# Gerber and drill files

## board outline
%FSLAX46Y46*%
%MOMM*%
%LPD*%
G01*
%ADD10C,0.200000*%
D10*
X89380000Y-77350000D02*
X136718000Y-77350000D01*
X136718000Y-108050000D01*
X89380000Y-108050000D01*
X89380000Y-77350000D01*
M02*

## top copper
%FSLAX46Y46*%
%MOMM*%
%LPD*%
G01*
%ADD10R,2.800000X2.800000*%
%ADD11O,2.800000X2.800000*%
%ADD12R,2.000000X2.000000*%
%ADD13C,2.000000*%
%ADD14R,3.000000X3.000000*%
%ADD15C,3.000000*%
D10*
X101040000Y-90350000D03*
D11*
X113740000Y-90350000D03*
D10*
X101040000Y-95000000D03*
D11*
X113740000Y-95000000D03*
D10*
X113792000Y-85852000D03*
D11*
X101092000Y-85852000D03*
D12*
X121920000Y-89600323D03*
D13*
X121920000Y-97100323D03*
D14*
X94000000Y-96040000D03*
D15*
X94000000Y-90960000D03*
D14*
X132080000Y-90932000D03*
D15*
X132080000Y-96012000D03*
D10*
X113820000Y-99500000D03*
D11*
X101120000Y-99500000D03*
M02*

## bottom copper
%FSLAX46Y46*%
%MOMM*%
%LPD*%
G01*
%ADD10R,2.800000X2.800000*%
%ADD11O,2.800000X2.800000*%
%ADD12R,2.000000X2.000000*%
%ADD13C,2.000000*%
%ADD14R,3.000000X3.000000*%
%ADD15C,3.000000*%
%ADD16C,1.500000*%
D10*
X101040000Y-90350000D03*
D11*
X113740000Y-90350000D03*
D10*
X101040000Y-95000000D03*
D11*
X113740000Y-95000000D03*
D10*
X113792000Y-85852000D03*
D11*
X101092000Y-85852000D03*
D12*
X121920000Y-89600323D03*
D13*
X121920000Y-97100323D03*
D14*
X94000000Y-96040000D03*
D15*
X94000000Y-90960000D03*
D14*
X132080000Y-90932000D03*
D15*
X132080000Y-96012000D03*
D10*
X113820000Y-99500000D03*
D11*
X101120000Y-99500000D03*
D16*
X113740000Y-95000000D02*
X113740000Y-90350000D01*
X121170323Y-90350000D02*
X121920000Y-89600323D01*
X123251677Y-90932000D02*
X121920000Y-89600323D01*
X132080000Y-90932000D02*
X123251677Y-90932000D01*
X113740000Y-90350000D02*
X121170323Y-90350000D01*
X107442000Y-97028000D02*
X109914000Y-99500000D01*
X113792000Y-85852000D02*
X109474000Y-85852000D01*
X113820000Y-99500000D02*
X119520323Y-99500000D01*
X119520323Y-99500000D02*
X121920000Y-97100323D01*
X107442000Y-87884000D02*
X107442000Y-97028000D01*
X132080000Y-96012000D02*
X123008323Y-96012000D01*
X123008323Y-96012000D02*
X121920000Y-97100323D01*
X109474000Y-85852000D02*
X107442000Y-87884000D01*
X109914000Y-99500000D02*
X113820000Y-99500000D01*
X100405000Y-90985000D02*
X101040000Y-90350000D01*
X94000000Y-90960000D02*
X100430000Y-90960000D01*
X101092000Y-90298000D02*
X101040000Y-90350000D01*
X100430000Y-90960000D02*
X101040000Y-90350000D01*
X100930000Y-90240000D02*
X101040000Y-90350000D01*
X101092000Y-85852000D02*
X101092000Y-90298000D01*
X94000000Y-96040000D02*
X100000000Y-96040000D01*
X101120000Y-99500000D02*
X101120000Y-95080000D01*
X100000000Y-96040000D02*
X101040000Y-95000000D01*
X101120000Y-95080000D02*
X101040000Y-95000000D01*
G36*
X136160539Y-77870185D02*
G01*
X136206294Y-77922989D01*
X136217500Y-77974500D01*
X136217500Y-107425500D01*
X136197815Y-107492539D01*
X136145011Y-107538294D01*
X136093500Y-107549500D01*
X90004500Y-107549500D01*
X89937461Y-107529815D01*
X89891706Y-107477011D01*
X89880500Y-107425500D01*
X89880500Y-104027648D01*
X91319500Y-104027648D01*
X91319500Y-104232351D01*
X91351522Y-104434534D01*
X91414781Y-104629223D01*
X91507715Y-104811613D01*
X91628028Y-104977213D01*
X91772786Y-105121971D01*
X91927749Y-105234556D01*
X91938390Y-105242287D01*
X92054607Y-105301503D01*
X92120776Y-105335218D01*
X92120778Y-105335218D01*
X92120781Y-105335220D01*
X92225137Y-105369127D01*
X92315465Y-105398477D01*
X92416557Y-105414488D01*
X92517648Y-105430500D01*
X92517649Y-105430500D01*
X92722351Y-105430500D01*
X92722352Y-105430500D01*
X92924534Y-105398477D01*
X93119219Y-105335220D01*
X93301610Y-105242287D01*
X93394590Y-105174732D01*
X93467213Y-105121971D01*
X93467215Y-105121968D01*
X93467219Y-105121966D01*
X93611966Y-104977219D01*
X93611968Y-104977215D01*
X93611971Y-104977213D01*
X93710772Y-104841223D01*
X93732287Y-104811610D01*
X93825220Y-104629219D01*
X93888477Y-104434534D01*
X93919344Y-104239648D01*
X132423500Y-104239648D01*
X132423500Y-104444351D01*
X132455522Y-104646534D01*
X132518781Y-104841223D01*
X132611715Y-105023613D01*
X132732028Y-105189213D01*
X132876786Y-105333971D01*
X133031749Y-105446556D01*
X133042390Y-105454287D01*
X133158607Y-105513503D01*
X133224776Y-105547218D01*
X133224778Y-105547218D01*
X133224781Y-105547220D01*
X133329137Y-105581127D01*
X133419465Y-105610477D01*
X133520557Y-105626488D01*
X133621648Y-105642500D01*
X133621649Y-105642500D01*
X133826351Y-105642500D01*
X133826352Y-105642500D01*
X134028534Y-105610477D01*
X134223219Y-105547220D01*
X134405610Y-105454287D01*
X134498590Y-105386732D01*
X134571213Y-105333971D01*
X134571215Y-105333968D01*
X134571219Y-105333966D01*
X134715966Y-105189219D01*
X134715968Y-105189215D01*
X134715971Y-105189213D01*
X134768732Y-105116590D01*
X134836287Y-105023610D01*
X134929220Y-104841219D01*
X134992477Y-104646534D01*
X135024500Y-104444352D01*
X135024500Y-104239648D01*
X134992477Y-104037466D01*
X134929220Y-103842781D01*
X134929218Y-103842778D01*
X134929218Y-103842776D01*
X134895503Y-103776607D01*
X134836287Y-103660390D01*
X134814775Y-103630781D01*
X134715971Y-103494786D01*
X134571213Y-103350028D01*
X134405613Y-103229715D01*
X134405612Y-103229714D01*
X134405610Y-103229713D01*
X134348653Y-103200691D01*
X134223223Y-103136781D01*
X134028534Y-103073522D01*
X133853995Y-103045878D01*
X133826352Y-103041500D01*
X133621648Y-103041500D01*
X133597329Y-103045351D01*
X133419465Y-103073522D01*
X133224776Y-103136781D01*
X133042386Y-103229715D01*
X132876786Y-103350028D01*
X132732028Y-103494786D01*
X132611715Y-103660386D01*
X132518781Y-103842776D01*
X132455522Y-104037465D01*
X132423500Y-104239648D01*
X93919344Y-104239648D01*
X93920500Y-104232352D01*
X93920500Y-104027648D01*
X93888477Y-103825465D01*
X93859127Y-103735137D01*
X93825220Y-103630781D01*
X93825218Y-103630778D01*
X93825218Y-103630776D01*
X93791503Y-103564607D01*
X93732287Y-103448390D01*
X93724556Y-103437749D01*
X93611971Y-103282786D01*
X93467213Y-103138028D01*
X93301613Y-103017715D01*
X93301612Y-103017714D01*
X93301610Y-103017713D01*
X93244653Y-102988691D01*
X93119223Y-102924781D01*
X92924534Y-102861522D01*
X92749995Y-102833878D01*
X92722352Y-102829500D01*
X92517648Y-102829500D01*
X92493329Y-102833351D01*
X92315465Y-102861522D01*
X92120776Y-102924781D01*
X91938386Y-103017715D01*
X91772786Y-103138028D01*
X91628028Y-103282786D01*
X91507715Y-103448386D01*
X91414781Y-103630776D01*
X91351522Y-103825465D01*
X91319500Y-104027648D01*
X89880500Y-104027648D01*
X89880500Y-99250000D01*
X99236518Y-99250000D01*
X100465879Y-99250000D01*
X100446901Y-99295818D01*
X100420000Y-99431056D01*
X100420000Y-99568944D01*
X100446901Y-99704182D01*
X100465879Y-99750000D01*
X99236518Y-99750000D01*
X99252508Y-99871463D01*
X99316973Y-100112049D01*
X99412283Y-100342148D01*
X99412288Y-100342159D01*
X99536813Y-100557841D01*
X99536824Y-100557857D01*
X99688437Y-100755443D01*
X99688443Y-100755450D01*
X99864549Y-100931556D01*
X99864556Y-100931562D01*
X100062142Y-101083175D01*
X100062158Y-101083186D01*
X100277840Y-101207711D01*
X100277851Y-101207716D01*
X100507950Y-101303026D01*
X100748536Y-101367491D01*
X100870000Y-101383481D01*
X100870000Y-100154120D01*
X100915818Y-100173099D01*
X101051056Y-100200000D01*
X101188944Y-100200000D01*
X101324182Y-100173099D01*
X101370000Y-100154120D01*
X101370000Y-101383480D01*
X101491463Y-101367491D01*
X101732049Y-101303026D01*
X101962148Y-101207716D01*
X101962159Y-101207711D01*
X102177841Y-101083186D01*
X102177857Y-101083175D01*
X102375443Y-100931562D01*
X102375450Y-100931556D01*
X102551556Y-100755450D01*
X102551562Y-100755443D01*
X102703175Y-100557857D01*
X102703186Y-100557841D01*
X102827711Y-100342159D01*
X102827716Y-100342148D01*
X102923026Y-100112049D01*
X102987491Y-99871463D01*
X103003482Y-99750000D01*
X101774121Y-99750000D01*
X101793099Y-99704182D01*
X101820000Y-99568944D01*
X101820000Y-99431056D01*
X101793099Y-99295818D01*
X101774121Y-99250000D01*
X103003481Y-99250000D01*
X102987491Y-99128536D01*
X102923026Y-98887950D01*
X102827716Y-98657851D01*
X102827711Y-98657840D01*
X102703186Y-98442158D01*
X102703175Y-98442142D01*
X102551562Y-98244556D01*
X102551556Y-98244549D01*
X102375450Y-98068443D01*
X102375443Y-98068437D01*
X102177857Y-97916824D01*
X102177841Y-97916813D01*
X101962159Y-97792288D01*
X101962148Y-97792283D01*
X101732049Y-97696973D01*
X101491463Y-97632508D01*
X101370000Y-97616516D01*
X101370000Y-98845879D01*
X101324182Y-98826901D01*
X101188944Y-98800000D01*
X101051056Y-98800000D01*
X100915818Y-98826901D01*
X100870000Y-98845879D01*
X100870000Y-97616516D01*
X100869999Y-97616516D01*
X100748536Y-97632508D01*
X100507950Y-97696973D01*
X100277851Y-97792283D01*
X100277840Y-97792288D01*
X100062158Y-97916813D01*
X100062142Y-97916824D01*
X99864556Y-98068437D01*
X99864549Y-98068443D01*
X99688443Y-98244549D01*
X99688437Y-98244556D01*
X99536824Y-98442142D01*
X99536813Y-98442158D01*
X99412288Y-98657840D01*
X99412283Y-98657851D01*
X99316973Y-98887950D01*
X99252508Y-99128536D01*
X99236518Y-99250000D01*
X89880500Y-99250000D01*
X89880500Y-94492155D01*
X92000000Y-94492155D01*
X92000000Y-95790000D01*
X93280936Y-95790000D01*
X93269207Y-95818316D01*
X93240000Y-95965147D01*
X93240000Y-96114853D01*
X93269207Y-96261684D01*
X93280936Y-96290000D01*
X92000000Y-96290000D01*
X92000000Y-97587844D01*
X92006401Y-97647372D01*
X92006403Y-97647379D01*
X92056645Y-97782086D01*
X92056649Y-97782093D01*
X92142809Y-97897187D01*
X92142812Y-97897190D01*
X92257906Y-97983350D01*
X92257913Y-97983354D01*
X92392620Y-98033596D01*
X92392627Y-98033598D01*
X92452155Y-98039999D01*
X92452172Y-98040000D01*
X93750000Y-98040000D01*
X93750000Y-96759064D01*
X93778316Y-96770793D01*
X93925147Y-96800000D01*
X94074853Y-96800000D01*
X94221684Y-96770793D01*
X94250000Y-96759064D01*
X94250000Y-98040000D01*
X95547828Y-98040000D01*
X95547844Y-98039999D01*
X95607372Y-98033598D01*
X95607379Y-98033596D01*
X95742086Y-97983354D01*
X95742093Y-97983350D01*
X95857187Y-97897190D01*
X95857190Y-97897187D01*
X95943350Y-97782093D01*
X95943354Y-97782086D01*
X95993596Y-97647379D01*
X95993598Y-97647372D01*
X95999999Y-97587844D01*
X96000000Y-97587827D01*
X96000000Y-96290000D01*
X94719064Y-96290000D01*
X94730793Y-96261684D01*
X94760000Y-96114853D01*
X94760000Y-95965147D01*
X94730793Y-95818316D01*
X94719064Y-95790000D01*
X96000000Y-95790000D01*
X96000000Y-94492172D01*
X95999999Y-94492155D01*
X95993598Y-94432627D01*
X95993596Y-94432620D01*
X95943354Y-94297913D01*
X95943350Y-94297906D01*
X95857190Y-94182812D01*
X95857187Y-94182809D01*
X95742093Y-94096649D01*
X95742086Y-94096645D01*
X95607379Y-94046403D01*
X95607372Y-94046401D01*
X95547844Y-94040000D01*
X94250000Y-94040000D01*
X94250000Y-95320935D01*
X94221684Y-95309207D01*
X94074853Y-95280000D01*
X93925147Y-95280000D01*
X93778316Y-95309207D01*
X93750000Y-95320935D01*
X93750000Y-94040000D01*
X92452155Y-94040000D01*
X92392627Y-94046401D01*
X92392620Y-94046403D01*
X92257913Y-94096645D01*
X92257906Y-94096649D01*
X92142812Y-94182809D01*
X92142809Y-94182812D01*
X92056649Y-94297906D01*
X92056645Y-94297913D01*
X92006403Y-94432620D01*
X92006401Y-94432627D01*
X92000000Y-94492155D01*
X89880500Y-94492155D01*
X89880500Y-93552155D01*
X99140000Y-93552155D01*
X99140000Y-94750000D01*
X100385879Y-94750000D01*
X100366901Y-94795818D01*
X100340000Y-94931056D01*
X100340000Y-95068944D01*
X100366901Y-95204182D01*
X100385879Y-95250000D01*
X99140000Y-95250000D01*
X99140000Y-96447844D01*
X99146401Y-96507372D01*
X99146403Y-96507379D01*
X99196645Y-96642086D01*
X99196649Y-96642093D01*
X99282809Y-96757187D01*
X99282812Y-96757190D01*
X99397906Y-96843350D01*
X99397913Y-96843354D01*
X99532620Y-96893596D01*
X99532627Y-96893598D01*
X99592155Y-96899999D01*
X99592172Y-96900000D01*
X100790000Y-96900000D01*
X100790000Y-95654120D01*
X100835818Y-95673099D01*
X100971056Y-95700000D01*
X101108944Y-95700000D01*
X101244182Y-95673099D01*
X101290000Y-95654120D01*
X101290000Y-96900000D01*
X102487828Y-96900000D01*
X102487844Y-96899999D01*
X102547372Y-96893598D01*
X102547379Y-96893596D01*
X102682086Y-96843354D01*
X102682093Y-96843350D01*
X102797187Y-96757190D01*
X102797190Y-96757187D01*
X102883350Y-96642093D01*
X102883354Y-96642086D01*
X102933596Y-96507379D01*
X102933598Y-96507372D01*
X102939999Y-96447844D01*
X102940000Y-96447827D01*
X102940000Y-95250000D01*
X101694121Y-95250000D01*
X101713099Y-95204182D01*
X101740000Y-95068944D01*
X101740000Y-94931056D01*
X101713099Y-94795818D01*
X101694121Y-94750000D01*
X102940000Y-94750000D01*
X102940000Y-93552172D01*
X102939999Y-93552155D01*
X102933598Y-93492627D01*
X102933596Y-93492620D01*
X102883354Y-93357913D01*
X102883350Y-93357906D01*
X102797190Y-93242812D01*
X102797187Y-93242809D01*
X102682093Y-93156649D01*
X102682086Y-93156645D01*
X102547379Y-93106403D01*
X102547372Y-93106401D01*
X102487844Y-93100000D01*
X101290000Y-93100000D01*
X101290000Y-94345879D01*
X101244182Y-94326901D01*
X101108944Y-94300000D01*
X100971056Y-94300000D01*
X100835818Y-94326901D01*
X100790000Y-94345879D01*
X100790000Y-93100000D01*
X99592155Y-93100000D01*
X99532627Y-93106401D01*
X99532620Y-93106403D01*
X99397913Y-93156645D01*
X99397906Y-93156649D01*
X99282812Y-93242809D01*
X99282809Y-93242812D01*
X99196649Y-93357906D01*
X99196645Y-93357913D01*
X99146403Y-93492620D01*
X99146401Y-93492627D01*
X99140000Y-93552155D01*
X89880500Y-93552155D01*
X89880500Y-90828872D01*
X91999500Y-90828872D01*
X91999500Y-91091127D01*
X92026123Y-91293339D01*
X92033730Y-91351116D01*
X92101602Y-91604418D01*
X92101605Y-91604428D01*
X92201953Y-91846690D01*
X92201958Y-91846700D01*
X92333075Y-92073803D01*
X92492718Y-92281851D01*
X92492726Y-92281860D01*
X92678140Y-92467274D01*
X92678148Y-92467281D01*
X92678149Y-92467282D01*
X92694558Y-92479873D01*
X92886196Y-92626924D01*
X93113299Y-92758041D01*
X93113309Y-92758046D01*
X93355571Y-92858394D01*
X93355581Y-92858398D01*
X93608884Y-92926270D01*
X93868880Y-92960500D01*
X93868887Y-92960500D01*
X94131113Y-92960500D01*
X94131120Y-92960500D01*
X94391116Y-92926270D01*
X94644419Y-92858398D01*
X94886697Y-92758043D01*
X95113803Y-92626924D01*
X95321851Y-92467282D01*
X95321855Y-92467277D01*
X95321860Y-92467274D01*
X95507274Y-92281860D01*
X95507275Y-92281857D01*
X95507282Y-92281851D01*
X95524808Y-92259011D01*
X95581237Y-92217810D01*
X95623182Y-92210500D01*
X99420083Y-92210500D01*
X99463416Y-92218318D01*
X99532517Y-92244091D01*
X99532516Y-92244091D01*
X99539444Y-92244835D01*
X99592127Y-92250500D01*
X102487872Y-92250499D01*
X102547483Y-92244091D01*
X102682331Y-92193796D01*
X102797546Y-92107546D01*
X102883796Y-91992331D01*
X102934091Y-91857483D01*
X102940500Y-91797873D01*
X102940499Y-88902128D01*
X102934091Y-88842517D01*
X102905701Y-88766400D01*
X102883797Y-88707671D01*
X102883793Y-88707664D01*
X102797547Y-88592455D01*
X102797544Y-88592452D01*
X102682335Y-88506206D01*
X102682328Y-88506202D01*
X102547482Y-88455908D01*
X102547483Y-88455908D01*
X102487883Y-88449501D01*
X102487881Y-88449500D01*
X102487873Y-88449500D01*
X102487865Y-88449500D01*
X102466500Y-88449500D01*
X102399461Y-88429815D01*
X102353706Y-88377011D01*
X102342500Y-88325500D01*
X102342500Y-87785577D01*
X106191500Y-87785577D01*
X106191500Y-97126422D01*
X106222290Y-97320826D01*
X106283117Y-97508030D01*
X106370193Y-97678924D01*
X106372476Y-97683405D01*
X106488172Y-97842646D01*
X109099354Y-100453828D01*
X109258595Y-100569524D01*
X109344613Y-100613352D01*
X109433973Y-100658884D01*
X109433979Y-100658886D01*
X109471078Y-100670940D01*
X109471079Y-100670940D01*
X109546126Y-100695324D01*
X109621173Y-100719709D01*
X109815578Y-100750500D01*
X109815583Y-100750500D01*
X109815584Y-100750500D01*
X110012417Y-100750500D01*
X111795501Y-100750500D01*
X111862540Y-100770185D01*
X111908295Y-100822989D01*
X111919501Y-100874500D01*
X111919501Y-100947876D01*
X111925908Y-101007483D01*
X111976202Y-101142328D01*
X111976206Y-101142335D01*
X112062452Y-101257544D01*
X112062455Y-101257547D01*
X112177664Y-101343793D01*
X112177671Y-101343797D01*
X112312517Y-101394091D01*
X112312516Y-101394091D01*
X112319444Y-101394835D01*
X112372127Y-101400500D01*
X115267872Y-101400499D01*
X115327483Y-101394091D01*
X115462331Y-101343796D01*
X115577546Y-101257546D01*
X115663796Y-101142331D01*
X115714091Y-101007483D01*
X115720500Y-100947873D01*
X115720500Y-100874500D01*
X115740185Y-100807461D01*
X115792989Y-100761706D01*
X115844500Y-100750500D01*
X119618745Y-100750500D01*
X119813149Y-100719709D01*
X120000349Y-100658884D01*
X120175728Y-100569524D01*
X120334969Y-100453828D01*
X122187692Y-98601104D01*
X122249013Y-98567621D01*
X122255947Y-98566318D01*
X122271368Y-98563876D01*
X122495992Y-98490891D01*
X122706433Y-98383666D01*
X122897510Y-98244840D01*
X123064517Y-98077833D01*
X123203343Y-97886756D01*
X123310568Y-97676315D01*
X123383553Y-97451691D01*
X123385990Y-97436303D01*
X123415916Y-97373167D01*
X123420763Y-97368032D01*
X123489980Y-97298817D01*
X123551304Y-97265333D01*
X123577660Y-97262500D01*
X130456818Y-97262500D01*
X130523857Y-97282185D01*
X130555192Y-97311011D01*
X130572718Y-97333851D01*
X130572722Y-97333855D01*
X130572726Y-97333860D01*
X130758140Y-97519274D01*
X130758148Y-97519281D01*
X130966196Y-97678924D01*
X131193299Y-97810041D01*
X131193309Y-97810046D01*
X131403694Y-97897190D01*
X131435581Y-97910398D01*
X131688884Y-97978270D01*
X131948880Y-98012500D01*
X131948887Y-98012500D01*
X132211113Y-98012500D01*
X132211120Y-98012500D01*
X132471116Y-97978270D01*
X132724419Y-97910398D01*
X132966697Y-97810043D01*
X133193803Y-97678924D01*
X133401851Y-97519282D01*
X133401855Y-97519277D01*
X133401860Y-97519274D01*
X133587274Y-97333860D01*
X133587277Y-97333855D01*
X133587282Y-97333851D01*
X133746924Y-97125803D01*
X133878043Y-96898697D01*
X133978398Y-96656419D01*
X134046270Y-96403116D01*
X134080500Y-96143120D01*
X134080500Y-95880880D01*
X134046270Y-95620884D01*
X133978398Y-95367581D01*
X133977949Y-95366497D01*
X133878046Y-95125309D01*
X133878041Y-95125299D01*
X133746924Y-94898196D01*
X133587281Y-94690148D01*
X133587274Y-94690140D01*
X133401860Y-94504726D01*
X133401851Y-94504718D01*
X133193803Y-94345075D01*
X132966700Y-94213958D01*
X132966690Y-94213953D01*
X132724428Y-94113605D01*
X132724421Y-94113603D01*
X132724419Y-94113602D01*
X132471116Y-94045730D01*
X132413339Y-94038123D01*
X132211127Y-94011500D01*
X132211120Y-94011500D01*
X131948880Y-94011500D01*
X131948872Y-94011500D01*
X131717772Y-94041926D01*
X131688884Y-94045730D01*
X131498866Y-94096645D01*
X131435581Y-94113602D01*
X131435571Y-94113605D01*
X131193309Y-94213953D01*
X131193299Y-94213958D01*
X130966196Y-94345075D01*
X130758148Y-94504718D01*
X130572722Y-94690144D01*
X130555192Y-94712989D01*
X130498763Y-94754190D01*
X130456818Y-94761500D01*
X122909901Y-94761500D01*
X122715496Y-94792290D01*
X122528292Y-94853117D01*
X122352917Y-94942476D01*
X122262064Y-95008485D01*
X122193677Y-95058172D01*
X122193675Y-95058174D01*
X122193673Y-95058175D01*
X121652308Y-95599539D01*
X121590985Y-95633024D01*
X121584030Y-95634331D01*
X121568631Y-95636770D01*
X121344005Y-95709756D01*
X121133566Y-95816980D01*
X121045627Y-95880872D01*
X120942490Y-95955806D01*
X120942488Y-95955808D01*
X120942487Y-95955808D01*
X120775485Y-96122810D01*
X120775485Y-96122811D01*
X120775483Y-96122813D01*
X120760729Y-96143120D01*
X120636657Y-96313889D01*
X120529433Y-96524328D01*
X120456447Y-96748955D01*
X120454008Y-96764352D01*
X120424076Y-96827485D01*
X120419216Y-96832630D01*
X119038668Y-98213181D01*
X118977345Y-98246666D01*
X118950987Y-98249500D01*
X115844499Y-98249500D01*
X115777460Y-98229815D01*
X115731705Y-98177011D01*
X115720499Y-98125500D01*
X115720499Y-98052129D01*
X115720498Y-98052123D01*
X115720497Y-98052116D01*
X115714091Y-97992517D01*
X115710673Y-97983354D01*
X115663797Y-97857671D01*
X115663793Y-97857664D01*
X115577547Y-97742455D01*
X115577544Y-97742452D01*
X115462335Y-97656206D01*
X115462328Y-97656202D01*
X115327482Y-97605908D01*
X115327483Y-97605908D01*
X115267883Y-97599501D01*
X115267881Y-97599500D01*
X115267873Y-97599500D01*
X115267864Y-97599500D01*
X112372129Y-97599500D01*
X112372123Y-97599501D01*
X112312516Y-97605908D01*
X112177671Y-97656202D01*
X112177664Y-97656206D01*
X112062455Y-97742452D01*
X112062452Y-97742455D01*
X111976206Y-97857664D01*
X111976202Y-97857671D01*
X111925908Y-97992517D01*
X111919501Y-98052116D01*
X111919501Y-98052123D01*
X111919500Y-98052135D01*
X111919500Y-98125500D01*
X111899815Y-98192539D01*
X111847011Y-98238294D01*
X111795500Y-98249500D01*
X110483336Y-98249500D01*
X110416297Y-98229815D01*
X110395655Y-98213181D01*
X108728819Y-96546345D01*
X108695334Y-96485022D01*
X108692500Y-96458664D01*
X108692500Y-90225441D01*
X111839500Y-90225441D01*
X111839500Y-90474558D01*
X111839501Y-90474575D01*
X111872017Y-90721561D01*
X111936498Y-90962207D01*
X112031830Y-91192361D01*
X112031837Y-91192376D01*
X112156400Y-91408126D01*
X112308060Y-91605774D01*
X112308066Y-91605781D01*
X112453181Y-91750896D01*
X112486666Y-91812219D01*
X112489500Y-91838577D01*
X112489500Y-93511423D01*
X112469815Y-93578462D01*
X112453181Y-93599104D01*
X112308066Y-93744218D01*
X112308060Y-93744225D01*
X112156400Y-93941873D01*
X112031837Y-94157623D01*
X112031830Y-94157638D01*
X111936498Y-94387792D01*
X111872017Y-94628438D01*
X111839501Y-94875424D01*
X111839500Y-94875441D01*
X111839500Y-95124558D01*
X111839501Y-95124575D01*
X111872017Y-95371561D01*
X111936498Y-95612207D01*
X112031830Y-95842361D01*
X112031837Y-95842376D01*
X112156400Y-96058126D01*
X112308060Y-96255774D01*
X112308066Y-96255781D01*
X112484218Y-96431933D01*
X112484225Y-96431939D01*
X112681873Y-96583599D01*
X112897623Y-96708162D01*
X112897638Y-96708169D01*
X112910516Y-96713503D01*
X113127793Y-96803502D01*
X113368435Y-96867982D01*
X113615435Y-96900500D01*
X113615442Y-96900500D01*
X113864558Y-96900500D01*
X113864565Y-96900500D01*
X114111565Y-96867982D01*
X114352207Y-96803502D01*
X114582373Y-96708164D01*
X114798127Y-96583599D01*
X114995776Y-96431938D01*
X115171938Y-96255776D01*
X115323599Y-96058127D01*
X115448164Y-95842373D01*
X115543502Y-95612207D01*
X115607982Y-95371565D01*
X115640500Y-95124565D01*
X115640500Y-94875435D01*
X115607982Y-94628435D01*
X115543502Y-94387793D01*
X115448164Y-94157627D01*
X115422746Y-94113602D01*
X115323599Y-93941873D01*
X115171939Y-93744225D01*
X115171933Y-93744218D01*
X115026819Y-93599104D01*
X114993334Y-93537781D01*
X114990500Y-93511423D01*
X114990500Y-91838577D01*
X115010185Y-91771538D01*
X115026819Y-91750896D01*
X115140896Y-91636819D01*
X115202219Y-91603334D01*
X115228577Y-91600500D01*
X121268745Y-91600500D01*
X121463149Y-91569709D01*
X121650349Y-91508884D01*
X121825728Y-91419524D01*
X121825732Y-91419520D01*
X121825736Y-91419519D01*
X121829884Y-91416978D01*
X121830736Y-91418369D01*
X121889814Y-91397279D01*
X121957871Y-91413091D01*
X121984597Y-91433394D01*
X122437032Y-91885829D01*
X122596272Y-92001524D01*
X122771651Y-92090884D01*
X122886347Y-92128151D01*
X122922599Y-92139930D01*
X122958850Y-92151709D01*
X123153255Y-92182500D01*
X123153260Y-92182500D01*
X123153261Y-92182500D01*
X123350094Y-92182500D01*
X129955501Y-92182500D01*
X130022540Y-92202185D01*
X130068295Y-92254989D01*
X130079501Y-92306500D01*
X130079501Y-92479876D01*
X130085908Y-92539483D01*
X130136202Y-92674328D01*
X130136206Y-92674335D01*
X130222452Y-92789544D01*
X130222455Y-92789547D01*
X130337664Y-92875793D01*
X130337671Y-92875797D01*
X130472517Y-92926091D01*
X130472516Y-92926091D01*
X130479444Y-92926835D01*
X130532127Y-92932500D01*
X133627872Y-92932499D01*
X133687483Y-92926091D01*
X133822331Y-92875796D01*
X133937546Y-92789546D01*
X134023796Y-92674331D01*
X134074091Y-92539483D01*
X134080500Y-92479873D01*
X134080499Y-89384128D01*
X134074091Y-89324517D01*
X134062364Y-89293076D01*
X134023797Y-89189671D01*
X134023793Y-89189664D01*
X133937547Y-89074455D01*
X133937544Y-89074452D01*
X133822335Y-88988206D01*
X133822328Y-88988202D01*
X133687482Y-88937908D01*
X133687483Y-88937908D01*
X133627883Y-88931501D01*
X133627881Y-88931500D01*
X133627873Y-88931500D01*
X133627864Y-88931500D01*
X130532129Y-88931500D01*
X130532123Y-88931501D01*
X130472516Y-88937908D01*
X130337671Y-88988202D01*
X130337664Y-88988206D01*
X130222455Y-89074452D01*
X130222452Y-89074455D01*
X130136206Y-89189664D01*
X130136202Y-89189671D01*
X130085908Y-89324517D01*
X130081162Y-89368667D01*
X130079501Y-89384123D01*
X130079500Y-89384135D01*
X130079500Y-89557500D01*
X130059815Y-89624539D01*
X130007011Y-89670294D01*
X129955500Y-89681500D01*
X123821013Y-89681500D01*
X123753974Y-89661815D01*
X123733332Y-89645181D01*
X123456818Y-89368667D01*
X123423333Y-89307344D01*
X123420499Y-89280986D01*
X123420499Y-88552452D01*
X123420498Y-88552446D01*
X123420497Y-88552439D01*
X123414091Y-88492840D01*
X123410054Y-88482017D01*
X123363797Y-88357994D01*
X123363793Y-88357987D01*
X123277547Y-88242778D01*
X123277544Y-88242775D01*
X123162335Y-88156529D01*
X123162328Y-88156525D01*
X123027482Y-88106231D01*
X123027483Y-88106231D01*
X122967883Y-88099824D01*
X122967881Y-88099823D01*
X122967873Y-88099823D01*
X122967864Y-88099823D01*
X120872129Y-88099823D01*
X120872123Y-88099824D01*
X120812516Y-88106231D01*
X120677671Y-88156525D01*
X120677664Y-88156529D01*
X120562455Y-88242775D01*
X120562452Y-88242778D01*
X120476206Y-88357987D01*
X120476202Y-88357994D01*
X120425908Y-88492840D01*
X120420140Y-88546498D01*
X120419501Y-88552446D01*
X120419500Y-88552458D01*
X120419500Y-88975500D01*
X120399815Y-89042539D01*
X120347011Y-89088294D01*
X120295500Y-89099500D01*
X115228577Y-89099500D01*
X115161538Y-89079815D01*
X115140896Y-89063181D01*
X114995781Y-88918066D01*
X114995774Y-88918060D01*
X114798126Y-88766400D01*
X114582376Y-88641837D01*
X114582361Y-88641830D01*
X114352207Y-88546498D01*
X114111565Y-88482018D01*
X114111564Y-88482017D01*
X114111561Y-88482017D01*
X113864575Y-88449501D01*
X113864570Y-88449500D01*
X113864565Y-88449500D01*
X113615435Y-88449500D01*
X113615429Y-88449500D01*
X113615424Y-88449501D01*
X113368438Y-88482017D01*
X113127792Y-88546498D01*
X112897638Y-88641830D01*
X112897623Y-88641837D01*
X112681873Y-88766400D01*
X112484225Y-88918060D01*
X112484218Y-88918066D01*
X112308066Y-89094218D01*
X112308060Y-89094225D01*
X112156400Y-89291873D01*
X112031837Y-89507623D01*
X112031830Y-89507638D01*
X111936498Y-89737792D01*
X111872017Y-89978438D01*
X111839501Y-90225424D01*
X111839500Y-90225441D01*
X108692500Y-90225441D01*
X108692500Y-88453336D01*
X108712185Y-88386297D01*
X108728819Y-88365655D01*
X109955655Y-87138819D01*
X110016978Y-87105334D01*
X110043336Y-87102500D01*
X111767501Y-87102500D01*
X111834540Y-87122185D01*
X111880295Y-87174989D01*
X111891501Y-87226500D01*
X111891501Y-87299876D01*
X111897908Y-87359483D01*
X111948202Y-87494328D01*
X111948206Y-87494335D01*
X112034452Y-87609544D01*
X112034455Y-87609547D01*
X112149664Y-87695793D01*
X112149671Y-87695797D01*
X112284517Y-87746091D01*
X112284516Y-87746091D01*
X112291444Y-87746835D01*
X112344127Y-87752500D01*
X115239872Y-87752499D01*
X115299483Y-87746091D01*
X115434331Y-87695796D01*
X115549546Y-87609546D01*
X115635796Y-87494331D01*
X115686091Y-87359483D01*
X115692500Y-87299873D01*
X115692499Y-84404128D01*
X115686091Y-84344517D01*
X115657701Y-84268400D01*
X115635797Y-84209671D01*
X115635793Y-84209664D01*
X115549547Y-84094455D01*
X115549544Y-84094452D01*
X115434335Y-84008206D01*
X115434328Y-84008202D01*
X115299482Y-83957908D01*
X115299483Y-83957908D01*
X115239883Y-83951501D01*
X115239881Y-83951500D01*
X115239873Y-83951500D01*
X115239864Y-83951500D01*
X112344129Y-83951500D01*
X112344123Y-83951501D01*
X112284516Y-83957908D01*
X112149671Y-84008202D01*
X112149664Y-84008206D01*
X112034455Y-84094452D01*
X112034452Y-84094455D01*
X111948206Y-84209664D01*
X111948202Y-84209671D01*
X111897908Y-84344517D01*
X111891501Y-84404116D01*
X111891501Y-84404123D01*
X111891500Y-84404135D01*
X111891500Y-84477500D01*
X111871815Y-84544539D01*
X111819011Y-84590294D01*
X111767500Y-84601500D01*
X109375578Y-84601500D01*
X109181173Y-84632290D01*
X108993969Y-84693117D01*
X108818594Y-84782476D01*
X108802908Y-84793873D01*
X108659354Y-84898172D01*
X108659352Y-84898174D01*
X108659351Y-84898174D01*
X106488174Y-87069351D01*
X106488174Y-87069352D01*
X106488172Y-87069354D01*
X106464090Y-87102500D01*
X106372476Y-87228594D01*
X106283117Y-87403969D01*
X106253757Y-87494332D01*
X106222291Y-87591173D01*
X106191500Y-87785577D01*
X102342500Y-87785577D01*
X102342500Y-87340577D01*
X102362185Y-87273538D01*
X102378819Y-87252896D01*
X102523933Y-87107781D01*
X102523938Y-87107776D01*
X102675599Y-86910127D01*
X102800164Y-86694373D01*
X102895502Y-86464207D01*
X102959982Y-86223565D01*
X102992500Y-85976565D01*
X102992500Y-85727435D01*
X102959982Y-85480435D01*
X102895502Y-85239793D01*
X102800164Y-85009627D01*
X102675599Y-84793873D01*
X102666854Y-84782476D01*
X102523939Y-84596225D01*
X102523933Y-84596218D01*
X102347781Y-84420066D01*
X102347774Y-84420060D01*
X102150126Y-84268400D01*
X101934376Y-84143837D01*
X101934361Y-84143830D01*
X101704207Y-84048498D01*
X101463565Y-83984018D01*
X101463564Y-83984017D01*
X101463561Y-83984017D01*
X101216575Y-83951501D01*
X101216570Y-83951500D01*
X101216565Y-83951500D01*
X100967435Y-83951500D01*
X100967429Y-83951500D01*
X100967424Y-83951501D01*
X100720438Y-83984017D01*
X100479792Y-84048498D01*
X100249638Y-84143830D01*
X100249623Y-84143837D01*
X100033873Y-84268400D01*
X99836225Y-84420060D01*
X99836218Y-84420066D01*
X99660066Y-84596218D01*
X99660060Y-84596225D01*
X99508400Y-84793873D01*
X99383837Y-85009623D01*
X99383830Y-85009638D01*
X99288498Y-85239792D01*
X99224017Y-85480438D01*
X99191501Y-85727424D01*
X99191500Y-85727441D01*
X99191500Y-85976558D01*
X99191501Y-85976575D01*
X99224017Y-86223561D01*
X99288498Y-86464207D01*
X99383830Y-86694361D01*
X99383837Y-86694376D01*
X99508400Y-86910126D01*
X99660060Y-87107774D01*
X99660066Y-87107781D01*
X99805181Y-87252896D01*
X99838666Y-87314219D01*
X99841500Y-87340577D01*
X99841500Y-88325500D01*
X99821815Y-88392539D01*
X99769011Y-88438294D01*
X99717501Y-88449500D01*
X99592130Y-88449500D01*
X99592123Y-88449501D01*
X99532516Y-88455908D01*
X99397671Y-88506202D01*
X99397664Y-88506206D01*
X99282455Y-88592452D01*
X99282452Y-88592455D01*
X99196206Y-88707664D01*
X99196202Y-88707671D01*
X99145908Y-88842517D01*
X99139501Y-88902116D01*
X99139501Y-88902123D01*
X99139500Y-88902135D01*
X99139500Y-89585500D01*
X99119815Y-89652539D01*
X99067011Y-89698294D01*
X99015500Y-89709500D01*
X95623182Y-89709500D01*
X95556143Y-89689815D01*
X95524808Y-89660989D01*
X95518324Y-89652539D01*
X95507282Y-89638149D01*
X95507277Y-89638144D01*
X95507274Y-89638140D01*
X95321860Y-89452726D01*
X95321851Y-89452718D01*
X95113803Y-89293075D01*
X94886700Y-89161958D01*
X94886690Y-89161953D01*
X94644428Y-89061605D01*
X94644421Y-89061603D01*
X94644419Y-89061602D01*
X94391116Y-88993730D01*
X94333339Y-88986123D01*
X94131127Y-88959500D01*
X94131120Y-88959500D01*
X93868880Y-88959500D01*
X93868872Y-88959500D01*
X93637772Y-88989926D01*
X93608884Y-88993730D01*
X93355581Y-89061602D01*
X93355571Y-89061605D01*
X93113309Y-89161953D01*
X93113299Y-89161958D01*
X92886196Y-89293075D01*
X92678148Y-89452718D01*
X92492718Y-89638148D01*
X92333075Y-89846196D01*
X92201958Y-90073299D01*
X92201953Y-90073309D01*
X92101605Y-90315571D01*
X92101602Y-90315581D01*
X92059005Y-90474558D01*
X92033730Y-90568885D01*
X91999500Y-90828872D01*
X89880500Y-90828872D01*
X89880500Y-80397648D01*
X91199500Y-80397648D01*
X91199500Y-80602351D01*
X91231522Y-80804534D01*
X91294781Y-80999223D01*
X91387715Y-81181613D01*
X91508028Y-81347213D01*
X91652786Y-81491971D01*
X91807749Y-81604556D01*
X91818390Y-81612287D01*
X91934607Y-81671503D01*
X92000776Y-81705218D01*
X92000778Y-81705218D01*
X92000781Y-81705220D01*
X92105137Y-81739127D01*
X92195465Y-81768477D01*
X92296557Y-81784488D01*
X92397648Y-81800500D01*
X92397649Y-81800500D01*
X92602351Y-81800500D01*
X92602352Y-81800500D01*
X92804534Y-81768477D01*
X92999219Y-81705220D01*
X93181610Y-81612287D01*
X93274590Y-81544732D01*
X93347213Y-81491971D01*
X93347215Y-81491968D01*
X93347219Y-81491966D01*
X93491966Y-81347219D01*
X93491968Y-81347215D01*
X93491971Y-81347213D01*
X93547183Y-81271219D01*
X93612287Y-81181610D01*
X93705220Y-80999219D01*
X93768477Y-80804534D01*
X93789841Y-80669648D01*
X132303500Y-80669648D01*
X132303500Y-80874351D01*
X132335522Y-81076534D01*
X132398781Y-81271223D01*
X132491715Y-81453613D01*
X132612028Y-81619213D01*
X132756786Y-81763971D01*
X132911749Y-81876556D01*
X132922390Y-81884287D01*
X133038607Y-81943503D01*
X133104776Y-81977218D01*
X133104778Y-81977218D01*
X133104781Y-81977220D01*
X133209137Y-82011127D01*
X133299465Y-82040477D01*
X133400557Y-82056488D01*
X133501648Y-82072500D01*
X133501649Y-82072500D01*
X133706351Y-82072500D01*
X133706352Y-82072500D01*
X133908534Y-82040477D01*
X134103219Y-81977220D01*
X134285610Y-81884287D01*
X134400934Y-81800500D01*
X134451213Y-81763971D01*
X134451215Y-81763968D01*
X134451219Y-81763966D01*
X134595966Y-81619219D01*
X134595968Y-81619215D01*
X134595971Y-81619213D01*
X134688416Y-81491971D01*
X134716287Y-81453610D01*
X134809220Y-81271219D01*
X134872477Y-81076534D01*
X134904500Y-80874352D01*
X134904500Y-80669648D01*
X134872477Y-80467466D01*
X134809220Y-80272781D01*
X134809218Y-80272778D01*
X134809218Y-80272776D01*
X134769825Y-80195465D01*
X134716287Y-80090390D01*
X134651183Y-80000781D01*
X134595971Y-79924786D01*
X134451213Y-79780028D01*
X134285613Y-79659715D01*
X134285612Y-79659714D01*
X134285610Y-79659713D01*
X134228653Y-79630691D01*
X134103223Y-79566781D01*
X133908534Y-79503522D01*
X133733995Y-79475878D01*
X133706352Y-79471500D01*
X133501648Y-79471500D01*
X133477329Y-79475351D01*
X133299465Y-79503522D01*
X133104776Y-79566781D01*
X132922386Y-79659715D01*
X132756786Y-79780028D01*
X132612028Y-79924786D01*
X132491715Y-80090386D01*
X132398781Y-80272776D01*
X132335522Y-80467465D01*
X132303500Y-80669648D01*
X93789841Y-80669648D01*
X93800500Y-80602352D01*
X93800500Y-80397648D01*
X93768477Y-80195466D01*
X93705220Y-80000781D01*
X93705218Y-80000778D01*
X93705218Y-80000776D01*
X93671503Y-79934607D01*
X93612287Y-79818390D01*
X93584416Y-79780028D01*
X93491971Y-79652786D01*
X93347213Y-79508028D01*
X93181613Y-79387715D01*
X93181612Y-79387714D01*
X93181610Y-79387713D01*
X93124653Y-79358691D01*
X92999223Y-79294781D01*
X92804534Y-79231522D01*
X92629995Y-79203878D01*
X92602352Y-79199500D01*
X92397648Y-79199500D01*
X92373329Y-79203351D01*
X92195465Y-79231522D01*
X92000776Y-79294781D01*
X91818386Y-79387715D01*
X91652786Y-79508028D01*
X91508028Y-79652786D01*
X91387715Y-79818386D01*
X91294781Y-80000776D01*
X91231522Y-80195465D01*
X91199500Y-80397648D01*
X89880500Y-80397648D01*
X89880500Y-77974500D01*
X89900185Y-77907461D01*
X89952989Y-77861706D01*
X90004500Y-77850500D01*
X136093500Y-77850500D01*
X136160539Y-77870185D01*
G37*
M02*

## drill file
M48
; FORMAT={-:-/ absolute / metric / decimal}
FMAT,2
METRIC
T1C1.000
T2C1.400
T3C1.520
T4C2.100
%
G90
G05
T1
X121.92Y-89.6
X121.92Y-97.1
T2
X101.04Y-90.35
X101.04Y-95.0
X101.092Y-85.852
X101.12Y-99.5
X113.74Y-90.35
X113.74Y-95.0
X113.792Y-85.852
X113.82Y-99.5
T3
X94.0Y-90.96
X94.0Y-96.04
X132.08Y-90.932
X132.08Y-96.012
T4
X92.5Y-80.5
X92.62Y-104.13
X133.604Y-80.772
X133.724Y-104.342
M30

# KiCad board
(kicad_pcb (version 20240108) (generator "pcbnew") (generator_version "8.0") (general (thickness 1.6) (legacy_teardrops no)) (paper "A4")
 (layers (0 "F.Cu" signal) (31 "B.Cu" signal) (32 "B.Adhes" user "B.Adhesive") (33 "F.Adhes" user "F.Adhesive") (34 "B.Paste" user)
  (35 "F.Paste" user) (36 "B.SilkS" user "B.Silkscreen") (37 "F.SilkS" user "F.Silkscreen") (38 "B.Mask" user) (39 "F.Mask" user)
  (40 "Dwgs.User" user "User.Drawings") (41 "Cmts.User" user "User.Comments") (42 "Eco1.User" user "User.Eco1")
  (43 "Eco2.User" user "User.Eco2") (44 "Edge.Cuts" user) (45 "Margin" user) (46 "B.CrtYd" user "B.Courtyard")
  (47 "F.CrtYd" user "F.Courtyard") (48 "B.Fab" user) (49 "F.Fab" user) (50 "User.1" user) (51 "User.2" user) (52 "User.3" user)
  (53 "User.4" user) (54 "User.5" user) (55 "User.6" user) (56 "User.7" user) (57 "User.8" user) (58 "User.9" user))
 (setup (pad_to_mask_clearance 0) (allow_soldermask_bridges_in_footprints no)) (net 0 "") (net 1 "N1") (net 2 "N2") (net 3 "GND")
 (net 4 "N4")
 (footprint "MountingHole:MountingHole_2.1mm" (layer "F.Cu") (at 133.604 80.772)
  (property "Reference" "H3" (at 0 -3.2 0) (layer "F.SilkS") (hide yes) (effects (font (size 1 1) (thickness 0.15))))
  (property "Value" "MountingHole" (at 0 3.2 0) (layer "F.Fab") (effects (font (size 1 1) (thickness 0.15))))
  (pad "" np_thru_hole circle (at 0 0) (size 2.1 2.1) (drill 2.1) (layers "*.Cu" "*.Mask")))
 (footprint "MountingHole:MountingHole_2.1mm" (layer "F.Cu") (at 92.5 80.5)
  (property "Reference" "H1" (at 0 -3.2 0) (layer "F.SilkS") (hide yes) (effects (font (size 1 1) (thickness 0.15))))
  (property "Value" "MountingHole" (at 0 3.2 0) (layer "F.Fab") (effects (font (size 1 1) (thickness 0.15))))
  (pad "" np_thru_hole circle (at 0 0) (size 2.1 2.1) (drill 2.1) (layers "*.Cu" "*.Mask")))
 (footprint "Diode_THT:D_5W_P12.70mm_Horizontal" (layer "F.Cu") (at 101.04 90.35)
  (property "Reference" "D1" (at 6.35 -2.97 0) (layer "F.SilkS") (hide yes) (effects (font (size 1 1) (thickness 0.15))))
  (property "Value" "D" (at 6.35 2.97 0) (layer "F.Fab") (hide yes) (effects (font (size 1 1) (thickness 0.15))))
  (pad "1" thru_hole rect (at 0 0) (size 2.8 2.8) (drill 1.4) (layers "*.Cu" "*.Mask") (remove_unused_layers no) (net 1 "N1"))
  (pad "2" thru_hole oval (at 12.7 0) (size 2.8 2.8) (drill 1.4) (layers "*.Cu" "*.Mask") (remove_unused_layers no) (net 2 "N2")))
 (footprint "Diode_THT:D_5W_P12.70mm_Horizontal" (layer "F.Cu") (at 101.04 95)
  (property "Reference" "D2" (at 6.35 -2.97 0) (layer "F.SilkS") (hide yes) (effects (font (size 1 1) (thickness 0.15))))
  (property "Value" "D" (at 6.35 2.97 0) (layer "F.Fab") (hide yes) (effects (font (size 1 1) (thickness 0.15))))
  (pad "1" thru_hole rect (at 0 0) (size 2.8 2.8) (drill 1.4) (layers "*.Cu" "*.Mask") (remove_unused_layers no) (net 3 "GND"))
  (pad "2" thru_hole oval (at 12.7 0) (size 2.8 2.8) (drill 1.4) (layers "*.Cu" "*.Mask") (remove_unused_layers no) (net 2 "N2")))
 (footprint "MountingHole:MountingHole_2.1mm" (layer "F.Cu") (at 92.62 104.13)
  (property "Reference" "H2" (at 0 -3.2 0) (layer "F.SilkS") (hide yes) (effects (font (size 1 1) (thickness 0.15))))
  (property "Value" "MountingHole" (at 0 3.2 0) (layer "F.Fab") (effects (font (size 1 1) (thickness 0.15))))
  (pad "" np_thru_hole circle (at 0 0) (size 2.1 2.1) (drill 2.1) (layers "*.Cu" "*.Mask")))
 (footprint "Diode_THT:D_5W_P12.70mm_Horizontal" (layer "F.Cu") (at 113.792 85.852 180)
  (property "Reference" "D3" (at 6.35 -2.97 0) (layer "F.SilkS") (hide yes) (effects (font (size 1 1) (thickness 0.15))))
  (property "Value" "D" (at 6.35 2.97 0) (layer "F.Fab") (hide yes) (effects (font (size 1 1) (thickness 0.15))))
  (pad "1" thru_hole rect (at 0 0 180) (size 2.8 2.8) (drill 1.4) (layers "*.Cu" "*.Mask") (remove_unused_layers no) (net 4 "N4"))
  (pad "2" thru_hole oval (at 12.7 0 180) (size 2.8 2.8) (drill 1.4) (layers "*.Cu" "*.Mask") (remove_unused_layers no) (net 1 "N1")))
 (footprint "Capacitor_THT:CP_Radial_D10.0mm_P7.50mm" (layer "F.Cu") (at 121.92 89.600323 -90)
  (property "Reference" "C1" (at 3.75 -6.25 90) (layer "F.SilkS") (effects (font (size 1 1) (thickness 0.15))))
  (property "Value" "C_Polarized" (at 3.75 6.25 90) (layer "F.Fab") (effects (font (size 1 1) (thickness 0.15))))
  (pad "1" thru_hole rect (at 0 0 270) (size 2 2) (drill 1) (layers "*.Cu" "*.Mask") (remove_unused_layers no) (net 2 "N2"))
  (pad "2" thru_hole circle (at 7.5 0 270) (size 2 2) (drill 1) (layers "*.Cu" "*.Mask") (remove_unused_layers no) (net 4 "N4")))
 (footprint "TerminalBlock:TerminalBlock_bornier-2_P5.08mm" (layer "F.Cu") (at 94 96.04 90)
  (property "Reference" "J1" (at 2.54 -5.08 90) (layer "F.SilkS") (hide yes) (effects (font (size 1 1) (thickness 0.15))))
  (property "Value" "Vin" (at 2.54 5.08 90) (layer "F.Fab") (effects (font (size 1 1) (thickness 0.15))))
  (pad "1" thru_hole rect (at 0 0 90) (size 3 3) (drill 1.52) (layers "*.Cu" "*.Mask") (remove_unused_layers no) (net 3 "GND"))
  (pad "2" thru_hole circle (at 5.08 0 90) (size 3 3) (drill 1.52) (layers "*.Cu" "*.Mask") (remove_unused_layers no) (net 1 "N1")))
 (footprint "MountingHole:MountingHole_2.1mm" (layer "F.Cu") (at 133.724 104.342)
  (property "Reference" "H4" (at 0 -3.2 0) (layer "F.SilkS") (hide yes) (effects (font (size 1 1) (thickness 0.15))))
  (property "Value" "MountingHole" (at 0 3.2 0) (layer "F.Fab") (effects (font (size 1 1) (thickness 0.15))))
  (pad "" np_thru_hole circle (at 0 0) (size 2.1 2.1) (drill 2.1) (layers "*.Cu" "*.Mask")))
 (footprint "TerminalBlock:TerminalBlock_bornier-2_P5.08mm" (layer "F.Cu") (at 132.08 90.932 -90)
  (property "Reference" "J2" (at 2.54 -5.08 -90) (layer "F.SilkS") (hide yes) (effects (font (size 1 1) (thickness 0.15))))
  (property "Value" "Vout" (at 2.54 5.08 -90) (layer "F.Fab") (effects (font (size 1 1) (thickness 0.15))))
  (pad "1" thru_hole rect (at 0 0 270) (size 3 3) (drill 1.52) (layers "*.Cu" "*.Mask") (remove_unused_layers no) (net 2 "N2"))
  (pad "2" thru_hole circle (at 5.08 0 270) (size 3 3) (drill 1.52) (layers "*.Cu" "*.Mask") (remove_unused_layers no) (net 4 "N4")))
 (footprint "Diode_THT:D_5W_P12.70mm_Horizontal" (layer "F.Cu") (at 113.82 99.5 180)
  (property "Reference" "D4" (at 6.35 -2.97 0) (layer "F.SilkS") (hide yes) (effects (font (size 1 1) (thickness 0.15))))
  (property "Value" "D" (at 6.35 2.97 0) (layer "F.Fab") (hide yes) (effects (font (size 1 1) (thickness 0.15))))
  (pad "1" thru_hole rect (at 0 0 180) (size 2.8 2.8) (drill 1.4) (layers "*.Cu" "*.Mask") (remove_unused_layers no) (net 4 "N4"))
  (pad "2" thru_hole oval (at 12.7 0 180) (size 2.8 2.8) (drill 1.4) (layers "*.Cu" "*.Mask") (remove_unused_layers no) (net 3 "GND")))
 (gr_rect (start 89.38 77.35) (end 136.718 108.05) (stroke (width 0.2) (type default)) (fill none) (layer "Edge.Cuts"))
 (segment (start 113.74 95) (end 113.74 90.35) (width 1.5) (layer "B.Cu") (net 2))
 (segment (start 121.170323 90.35) (end 121.92 89.600323) (width 1.5) (layer "B.Cu") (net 2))
 (segment (start 123.251677 90.932) (end 121.92 89.600323) (width 1.5) (layer "B.Cu") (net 2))
 (segment (start 132.08 90.932) (end 123.251677 90.932) (width 1.5) (layer "B.Cu") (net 2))
 (segment (start 113.74 90.35) (end 121.170323 90.35) (width 1.5) (layer "B.Cu") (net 2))
 (segment (start 107.442 97.028) (end 109.914 99.5) (width 1.5) (layer "B.Cu") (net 4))
 (segment (start 113.792 85.852) (end 109.474 85.852) (width 1.5) (layer "B.Cu") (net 4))
 (segment (start 113.82 99.5) (end 119.520323 99.5) (width 1.5) (layer "B.Cu") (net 4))
 (segment (start 119.520323 99.5) (end 121.92 97.100323) (width 1.5) (layer "B.Cu") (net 4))
 (segment (start 107.442 87.884) (end 107.442 97.028) (width 1.5) (layer "B.Cu") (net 4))
 (segment (start 132.08 96.012) (end 123.008323 96.012) (width 1.5) (layer "B.Cu") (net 4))
 (segment (start 123.008323 96.012) (end 121.92 97.100323) (width 1.5) (layer "B.Cu") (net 4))
 (segment (start 109.474 85.852) (end 107.442 87.884) (width 1.5) (layer "B.Cu") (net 4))
 (segment (start 109.914 99.5) (end 113.82 99.5) (width 1.5) (layer "B.Cu") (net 4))
 (segment (start 100.405 90.985) (end 101.04 90.35) (width 1.5) (layer "B.Cu") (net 1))
 (segment (start 94 90.96) (end 100.43 90.96) (width 1.5) (layer "B.Cu") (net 1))
 (segment (start 101.092 90.298) (end 101.04 90.35) (width 1.5) (layer "B.Cu") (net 1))
 (segment (start 100.43 90.96) (end 101.04 90.35) (width 1.5) (layer "B.Cu") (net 1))
 (segment (start 100.93 90.24) (end 101.04 90.35) (width 1.5) (layer "B.Cu") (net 1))
 (segment (start 101.092 85.852) (end 101.092 90.298) (width 1.5) (layer "B.Cu") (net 1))
 (segment (start 94 96.04) (end 100 96.04) (width 1.5) (layer "B.Cu") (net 3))
 (segment (start 101.12 99.5) (end 101.12 95.08) (width 1.5) (layer "B.Cu") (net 3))
 (segment (start 100 96.04) (end 101.04 95) (width 1.5) (layer "B.Cu") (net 3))
 (segment (start 101.12 95.08) (end 101.04 95) (width 1.5) (layer "B.Cu") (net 3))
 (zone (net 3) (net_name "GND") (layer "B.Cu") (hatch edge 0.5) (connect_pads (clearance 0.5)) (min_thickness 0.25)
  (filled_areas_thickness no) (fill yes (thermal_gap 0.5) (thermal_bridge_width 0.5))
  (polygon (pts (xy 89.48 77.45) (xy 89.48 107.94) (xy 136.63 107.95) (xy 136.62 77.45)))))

